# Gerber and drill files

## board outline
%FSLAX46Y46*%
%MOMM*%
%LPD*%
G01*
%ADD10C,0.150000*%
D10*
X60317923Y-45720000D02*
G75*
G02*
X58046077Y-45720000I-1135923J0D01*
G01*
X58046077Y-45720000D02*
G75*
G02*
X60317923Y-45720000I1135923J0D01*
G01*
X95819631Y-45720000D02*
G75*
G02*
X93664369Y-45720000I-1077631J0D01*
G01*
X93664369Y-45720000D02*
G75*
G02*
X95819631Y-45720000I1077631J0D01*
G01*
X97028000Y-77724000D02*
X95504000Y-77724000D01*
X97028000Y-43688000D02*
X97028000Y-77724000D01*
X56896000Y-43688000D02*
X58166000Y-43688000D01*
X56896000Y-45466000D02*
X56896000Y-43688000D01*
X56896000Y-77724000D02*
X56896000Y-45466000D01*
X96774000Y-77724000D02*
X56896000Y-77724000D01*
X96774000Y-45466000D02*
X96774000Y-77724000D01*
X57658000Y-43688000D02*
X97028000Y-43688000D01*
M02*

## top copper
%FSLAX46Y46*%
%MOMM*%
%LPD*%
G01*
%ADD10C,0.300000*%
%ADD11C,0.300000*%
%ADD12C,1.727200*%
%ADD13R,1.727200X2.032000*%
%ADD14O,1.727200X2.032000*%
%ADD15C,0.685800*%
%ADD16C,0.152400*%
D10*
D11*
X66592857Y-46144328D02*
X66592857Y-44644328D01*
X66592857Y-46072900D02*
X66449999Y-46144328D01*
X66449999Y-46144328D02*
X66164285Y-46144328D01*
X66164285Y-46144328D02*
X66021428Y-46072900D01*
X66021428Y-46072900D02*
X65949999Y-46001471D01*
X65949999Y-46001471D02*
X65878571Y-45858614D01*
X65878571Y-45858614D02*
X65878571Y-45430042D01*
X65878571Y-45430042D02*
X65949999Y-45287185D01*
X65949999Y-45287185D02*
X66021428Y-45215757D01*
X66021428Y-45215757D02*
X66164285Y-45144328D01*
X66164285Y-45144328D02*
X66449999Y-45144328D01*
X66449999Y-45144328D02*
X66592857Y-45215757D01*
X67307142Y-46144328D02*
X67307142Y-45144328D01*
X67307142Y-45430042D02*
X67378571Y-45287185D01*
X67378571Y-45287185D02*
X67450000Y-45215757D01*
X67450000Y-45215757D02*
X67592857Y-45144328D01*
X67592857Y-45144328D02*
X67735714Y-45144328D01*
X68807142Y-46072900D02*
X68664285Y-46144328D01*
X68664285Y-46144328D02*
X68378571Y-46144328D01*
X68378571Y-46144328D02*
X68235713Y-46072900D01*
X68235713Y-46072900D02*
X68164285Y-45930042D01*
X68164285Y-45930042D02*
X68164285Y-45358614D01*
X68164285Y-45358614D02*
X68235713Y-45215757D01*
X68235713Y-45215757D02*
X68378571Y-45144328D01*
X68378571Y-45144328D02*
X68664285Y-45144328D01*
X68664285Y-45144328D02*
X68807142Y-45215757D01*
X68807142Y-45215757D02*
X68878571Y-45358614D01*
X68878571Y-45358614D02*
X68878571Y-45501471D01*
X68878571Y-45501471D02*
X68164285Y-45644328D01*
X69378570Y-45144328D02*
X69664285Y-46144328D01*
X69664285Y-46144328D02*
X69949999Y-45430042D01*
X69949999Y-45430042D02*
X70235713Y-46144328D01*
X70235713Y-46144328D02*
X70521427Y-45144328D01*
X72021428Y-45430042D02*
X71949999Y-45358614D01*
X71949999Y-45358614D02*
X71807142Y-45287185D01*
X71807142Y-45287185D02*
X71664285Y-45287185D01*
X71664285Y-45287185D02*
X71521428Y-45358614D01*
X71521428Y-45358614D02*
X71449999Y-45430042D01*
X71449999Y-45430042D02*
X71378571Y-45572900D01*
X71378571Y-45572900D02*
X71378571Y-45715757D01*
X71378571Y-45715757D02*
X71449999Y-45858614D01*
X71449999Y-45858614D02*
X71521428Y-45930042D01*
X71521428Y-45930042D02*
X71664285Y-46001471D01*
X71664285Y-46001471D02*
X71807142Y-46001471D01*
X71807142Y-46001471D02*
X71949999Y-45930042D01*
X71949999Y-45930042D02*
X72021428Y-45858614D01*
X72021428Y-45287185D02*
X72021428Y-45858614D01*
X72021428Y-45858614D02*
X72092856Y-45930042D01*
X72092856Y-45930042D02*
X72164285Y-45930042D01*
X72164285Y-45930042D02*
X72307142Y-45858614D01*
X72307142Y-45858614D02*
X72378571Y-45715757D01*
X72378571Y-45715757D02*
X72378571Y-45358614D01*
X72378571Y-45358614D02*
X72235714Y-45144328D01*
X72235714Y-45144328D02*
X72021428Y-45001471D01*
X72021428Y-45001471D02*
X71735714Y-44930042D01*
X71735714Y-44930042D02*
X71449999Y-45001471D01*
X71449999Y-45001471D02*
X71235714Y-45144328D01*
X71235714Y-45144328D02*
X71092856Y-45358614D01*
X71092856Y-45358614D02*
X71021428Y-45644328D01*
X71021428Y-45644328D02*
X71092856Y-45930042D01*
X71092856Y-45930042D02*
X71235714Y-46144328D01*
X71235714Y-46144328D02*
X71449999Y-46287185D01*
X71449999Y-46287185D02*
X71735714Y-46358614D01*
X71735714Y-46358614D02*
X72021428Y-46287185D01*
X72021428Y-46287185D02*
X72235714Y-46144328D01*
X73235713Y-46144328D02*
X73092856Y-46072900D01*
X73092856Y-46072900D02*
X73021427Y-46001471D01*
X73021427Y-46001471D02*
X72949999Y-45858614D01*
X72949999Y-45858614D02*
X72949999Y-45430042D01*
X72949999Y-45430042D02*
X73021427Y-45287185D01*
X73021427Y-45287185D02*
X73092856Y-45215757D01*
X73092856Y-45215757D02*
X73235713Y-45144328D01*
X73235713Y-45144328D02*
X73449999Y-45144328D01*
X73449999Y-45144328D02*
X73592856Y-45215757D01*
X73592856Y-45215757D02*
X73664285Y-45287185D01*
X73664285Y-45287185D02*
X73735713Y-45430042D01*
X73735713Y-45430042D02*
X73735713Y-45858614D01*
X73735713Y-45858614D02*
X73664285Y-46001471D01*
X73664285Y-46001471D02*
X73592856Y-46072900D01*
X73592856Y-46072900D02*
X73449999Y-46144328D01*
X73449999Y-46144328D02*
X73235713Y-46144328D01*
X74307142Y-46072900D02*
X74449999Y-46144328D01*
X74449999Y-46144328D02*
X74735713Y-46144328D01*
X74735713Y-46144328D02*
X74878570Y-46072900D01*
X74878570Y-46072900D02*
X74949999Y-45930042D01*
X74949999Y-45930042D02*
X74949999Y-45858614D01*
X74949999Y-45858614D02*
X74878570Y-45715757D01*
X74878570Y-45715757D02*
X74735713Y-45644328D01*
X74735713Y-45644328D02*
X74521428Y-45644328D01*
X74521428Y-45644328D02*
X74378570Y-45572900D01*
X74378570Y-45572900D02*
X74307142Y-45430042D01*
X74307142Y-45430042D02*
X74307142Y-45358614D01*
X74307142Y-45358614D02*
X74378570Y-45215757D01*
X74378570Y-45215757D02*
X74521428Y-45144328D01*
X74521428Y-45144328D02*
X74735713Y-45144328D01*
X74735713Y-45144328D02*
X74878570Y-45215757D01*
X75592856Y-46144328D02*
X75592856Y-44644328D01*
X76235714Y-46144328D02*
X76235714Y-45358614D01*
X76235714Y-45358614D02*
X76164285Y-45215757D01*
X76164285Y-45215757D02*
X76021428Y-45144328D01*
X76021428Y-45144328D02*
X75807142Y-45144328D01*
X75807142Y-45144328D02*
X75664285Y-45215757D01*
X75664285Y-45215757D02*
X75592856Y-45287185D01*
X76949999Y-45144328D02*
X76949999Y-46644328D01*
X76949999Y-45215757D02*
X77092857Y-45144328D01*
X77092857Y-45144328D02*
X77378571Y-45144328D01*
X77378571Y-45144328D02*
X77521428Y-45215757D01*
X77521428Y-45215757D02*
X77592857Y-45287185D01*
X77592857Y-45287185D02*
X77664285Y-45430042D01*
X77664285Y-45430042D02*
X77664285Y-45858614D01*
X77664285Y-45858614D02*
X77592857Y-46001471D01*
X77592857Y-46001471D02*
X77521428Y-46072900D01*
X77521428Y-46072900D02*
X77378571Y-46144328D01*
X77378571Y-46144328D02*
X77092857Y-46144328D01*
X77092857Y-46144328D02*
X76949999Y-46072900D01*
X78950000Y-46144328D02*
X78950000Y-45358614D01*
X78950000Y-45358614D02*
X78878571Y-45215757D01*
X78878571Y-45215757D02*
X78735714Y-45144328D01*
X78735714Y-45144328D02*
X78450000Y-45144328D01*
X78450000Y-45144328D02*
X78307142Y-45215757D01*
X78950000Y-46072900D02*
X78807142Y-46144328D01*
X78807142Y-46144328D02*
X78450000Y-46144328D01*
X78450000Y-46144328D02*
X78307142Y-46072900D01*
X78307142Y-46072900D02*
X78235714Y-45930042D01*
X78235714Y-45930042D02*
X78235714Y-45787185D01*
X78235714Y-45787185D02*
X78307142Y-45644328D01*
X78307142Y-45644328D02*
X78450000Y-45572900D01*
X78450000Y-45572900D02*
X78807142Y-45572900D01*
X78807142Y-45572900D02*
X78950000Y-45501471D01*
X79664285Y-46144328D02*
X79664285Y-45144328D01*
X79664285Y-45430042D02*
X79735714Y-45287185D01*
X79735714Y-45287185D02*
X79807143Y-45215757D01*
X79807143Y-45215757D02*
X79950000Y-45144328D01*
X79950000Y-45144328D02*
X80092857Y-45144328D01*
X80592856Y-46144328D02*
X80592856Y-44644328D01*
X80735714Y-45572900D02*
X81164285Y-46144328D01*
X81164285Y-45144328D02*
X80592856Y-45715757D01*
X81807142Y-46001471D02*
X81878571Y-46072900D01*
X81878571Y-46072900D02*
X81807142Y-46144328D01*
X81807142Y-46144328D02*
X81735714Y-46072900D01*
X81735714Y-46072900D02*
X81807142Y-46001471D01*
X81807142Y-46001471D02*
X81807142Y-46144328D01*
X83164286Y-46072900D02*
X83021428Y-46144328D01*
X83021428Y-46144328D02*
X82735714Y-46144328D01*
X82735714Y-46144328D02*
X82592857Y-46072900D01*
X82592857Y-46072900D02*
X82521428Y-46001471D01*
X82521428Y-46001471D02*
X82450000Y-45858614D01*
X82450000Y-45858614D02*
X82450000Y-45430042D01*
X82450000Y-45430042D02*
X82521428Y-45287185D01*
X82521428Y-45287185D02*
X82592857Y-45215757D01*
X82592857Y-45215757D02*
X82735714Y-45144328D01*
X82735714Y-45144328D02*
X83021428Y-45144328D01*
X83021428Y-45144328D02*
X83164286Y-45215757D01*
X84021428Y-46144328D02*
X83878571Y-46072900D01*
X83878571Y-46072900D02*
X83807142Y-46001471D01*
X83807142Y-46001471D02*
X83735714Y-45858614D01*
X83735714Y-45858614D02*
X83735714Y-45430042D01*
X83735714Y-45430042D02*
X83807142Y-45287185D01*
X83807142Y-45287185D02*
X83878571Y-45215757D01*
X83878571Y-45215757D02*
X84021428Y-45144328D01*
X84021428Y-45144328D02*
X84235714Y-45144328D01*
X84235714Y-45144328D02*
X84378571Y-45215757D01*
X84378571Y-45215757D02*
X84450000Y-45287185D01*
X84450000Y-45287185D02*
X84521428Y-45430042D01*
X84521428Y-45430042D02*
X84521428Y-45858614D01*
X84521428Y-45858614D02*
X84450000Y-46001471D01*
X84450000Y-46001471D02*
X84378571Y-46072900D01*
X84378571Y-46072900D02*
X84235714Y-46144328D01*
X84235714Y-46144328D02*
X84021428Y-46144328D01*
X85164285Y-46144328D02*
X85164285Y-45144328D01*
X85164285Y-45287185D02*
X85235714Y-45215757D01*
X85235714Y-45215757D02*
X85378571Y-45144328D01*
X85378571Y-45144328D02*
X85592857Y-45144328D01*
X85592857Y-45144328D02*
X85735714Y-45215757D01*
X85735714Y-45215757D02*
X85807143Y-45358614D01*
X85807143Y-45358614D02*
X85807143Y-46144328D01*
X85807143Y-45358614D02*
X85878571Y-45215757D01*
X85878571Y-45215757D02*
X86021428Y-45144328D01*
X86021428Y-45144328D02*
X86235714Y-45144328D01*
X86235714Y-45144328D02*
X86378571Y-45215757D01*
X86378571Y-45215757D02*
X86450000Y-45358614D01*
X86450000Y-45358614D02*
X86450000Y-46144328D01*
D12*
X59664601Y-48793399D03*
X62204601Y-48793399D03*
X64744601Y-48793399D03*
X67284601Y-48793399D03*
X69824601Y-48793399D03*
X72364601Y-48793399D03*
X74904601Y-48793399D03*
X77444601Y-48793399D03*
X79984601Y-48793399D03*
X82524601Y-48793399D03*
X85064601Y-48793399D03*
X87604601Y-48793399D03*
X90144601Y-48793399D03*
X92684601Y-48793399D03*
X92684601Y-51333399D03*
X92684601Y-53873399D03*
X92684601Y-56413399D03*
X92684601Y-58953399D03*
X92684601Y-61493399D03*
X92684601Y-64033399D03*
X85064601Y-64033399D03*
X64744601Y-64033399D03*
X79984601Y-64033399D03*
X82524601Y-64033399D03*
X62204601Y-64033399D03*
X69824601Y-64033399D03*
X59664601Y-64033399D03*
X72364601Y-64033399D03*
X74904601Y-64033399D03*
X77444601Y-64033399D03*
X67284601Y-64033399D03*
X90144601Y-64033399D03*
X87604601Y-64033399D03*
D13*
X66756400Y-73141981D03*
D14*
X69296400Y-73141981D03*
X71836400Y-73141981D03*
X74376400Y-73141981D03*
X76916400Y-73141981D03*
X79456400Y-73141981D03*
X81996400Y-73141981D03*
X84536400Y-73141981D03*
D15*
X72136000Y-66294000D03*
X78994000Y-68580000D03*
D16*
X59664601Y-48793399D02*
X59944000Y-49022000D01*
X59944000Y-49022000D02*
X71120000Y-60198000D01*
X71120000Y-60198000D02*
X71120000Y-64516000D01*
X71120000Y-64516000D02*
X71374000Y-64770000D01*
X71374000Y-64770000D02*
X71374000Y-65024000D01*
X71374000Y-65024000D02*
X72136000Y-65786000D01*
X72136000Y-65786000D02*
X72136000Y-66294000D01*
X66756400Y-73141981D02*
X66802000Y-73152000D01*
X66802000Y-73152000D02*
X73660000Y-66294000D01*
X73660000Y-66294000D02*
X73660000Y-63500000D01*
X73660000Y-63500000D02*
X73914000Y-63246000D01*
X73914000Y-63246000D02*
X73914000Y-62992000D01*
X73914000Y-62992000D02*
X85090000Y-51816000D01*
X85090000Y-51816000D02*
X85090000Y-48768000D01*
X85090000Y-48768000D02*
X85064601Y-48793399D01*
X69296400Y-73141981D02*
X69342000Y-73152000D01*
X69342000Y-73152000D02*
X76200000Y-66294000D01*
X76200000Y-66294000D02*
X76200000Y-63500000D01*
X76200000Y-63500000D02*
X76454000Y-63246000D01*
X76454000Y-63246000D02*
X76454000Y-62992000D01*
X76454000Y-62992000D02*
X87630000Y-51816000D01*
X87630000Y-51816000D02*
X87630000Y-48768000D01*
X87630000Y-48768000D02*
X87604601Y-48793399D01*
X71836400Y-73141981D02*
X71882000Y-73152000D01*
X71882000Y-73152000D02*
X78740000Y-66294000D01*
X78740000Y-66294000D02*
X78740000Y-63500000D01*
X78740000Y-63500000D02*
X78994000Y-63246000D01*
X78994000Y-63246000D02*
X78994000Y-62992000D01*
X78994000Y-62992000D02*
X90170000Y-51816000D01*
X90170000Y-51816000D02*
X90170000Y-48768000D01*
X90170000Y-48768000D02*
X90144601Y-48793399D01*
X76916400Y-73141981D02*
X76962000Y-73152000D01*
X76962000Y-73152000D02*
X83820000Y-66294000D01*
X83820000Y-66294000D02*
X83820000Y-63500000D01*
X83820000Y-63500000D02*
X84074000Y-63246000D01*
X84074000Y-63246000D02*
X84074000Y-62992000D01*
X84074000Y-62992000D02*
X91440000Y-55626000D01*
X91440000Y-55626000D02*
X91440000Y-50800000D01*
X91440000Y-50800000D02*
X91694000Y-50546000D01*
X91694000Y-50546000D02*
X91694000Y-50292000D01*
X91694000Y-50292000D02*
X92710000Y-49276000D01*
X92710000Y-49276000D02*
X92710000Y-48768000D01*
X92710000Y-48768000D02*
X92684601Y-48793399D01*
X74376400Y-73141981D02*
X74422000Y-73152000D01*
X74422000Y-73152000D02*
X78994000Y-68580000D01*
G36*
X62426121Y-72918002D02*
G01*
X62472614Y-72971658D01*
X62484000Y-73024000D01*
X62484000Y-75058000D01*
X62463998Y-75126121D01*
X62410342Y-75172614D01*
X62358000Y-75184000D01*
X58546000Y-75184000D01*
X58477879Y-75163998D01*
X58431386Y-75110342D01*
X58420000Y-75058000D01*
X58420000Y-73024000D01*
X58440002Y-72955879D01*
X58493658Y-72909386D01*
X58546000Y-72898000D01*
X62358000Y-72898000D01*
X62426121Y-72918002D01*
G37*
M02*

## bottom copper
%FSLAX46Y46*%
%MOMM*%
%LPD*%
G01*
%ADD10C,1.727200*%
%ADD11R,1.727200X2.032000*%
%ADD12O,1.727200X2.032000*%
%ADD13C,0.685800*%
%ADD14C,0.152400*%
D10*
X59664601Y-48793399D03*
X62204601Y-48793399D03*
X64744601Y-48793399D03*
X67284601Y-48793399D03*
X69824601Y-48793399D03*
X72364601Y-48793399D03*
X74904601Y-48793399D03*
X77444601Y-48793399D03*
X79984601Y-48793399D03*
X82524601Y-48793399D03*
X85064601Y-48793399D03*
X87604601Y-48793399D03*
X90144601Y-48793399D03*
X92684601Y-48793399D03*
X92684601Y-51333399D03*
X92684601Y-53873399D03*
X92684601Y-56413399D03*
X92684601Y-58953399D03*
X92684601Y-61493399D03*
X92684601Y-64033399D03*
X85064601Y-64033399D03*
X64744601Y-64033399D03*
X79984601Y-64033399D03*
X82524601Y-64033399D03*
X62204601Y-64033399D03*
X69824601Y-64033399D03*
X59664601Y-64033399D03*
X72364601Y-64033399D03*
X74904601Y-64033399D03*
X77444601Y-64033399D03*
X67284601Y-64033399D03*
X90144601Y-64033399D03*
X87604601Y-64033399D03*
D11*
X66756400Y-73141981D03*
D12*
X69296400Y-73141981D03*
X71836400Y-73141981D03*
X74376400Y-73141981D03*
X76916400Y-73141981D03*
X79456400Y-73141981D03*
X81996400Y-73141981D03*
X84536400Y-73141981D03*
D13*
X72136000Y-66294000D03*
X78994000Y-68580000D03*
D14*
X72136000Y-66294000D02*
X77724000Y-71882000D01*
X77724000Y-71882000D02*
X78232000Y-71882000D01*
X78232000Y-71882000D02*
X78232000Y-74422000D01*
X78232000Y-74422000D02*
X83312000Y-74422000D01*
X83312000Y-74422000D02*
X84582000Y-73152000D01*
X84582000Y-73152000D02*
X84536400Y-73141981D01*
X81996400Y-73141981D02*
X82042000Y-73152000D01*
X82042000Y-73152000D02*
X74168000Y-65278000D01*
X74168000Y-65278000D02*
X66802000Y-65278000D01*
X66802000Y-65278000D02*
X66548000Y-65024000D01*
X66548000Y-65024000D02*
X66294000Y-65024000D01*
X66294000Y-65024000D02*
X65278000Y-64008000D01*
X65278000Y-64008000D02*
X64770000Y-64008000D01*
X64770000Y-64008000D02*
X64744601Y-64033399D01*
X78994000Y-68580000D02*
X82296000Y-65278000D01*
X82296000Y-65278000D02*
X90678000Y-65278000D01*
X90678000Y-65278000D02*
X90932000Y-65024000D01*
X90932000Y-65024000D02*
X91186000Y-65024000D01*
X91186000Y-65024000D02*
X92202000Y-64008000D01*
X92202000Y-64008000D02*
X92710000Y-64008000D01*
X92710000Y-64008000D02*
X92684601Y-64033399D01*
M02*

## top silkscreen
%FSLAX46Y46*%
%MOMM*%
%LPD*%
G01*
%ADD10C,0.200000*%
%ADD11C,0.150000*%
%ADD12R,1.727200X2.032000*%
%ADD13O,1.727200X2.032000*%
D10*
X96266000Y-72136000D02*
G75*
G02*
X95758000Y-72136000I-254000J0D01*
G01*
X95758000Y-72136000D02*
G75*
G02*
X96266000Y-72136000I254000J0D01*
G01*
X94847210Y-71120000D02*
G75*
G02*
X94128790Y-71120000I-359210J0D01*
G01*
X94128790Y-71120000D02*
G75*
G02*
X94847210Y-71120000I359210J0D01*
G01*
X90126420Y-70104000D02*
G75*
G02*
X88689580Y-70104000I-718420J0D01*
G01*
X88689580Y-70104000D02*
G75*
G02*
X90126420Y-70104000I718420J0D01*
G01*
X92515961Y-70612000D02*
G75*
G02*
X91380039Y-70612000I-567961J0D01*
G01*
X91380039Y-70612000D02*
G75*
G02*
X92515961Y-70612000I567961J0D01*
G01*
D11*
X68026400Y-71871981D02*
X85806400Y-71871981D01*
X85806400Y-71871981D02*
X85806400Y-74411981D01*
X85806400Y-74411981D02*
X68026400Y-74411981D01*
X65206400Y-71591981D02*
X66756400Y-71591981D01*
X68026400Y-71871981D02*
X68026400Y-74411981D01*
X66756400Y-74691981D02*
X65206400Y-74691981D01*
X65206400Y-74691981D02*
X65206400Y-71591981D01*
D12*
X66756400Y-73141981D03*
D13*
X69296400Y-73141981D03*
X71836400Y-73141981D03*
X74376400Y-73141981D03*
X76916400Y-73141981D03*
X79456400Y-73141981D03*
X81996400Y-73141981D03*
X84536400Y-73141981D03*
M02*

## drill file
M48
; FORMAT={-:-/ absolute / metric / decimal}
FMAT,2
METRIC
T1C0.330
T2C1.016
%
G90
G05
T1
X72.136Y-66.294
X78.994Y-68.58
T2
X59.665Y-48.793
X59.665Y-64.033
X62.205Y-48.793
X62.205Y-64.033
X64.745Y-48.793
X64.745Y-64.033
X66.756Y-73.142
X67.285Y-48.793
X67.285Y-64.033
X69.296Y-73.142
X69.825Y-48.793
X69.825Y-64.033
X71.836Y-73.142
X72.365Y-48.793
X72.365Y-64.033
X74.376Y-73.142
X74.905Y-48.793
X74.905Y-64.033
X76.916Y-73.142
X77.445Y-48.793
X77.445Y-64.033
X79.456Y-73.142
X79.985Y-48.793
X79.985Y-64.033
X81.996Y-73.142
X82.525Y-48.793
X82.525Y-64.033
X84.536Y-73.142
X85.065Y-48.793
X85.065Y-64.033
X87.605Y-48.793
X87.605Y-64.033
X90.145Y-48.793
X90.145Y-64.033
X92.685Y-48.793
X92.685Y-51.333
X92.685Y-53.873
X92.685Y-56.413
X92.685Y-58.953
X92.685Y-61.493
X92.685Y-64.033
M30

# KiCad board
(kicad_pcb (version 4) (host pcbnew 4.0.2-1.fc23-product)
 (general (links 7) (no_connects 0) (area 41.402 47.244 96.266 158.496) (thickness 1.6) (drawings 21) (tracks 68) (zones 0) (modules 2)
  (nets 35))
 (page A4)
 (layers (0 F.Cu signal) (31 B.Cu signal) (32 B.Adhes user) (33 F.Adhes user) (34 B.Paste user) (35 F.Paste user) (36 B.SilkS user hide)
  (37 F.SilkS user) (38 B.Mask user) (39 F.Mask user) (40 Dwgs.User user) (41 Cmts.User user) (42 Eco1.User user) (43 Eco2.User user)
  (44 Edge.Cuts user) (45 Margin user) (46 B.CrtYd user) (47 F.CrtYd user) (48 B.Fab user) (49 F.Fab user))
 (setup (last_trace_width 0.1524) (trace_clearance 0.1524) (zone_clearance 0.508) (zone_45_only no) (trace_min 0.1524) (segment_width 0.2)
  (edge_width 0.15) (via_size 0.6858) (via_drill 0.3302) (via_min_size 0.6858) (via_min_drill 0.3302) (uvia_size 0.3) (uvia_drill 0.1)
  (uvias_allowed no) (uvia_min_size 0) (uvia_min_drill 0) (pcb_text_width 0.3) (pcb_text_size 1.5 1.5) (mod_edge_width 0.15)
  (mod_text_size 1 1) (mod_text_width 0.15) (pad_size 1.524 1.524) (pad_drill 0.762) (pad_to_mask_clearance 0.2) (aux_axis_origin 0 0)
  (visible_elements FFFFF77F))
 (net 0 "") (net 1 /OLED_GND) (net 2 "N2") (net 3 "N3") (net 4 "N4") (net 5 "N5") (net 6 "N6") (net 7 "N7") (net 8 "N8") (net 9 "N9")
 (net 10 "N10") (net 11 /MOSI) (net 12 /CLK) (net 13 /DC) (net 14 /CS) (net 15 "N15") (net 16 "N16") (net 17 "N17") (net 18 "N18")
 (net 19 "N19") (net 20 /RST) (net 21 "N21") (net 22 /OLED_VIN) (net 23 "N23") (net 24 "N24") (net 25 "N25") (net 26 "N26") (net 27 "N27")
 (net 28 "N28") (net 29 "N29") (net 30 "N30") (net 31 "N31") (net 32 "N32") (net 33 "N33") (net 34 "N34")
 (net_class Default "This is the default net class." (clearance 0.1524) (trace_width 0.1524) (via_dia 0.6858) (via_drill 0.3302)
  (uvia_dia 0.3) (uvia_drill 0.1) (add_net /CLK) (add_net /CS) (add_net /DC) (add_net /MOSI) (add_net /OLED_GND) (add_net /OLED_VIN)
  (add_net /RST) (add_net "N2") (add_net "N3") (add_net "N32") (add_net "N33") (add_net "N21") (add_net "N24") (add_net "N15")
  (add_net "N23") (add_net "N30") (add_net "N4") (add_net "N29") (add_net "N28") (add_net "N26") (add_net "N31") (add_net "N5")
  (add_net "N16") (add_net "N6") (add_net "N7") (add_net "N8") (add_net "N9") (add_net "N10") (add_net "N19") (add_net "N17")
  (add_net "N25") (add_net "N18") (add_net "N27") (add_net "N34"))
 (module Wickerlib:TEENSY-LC (layer B.Cu) (at 69.824601 58.953399 270)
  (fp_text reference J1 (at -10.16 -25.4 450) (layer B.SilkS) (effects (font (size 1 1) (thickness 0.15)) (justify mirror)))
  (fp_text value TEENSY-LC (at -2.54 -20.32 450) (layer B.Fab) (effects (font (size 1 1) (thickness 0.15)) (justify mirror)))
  (pad G1 thru_hole circle (at -10.16 10.16 270) (size 1.7272 1.7272) (drill 1.016) (layers *.Cu *.Mask B.SilkS) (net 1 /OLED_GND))
  (pad 0 thru_hole circle (at -10.16 7.62 270) (size 1.7272 1.7272) (drill 1.016) (layers *.Cu *.Mask B.SilkS) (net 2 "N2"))
  (pad 1 thru_hole circle (at -10.16 5.08 270) (size 1.7272 1.7272) (drill 1.016) (layers *.Cu *.Mask B.SilkS) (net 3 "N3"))
  (pad 2 thru_hole circle (at -10.16 2.54 270) (size 1.7272 1.7272) (drill 1.016) (layers *.Cu *.Mask B.SilkS) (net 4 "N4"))
  (pad 3 thru_hole circle (at -10.16 0 270) (size 1.7272 1.7272) (drill 1.016) (layers *.Cu *.Mask B.SilkS) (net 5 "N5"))
  (pad 4 thru_hole circle (at -10.16 -2.54 270) (size 1.7272 1.7272) (drill 1.016) (layers *.Cu *.Mask B.SilkS) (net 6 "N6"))
  (pad 5 thru_hole circle (at -10.16 -5.08 270) (size 1.7272 1.7272) (drill 1.016) (layers *.Cu *.Mask B.SilkS) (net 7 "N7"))
  (pad 6 thru_hole circle (at -10.16 -7.62 270) (size 1.7272 1.7272) (drill 1.016) (layers *.Cu *.Mask B.SilkS) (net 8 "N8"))
  (pad 7 thru_hole circle (at -10.16 -10.16 270) (size 1.7272 1.7272) (drill 1.016) (layers *.Cu *.Mask B.SilkS) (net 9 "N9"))
  (pad 8 thru_hole circle (at -10.16 -12.7 270) (size 1.7272 1.7272) (drill 1.016) (layers *.Cu *.Mask B.SilkS) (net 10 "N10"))
  (pad 9 thru_hole circle (at -10.16 -15.24 270) (size 1.7272 1.7272) (drill 1.016) (layers *.Cu *.Mask B.SilkS) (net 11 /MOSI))
  (pad 10 thru_hole circle (at -10.16 -17.78 270) (size 1.7272 1.7272) (drill 1.016) (layers *.Cu *.Mask B.SilkS) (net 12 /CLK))
  (pad 11 thru_hole circle (at -10.16 -20.32 270) (size 1.7272 1.7272) (drill 1.016) (layers *.Cu *.Mask B.SilkS) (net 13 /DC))
  (pad 12 thru_hole circle (at -10.16 -22.86 270) (size 1.7272 1.7272) (drill 1.016) (layers *.Cu *.Mask B.SilkS) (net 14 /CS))
  (pad 17A thru_hole circle (at -7.62 -22.86 270) (size 1.7272 1.7272) (drill 1.016) (layers *.Cu *.Mask B.SilkS) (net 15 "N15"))
  (pad 3V1 thru_hole circle (at -5.08 -22.86 270) (size 1.7272 1.7272) (drill 1.016) (layers *.Cu *.Mask B.SilkS) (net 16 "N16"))
  (pad G2 thru_hole circle (at -2.54 -22.86 270) (size 1.7272 1.7272) (drill 1.016) (layers *.Cu *.Mask B.SilkS) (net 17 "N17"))
  (pad PGM thru_hole circle (at 0 -22.86 270) (size 1.7272 1.7272) (drill 1.016) (layers *.Cu *.Mask B.SilkS) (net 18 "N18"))
  (pad DAC thru_hole circle (at 2.54 -22.86 270) (size 1.7272 1.7272) (drill 1.016) (layers *.Cu *.Mask B.SilkS) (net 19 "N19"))
  (pad 13 thru_hole circle (at 5.08 -22.86 270) (size 1.7272 1.7272) (drill 1.016) (layers *.Cu *.Mask B.SilkS) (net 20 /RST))
  (pad 16 thru_hole circle (at 5.08 -15.24 270) (size 1.7272 1.7272) (drill 1.016) (layers *.Cu *.Mask B.SilkS) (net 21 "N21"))
  (pad 3V2 thru_hole circle (at 5.08 5.08 270) (size 1.7272 1.7272) (drill 1.016) (layers *.Cu *.Mask B.SilkS) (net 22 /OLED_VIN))
  (pad 18 thru_hole circle (at 5.08 -10.16 270) (size 1.7272 1.7272) (drill 1.016) (layers *.Cu *.Mask B.SilkS) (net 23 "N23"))
  (pad 17 thru_hole circle (at 5.08 -12.7 270) (size 1.7272 1.7272) (drill 1.016) (layers *.Cu *.Mask B.SilkS) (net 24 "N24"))
  (pad G3 thru_hole circle (at 5.08 7.62 270) (size 1.7272 1.7272) (drill 1.016) (layers *.Cu *.Mask B.SilkS) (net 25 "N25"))
  (pad 22 thru_hole circle (at 5.08 0 270) (size 1.7272 1.7272) (drill 1.016) (layers *.Cu *.Mask B.SilkS) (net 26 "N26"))
  (pad VIN thru_hole circle (at 5.08 10.16 270) (size 1.7272 1.7272) (drill 1.016) (layers *.Cu *.Mask B.SilkS) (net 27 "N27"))
  (pad 21 thru_hole circle (at 5.08 -2.54 270) (size 1.7272 1.7272) (drill 1.016) (layers *.Cu *.Mask B.SilkS) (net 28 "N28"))
  (pad 20 thru_hole circle (at 5.08 -5.08 270) (size 1.7272 1.7272) (drill 1.016) (layers *.Cu *.Mask B.SilkS) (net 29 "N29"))
  (pad 19 thru_hole circle (at 5.08 -7.62 270) (size 1.7272 1.7272) (drill 1.016) (layers *.Cu *.Mask B.SilkS) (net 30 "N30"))
  (pad 23 thru_hole circle (at 5.08 2.54 270) (size 1.7272 1.7272) (drill 1.016) (layers *.Cu *.Mask B.SilkS) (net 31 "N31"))
  (pad 14 thru_hole circle (at 5.08 -20.32 270) (size 1.7272 1.7272) (drill 1.016) (layers *.Cu *.Mask B.SilkS) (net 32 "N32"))
  (pad 15 thru_hole circle (at 5.08 -17.78 270) (size 1.7272 1.7272) (drill 1.016) (layers *.Cu *.Mask B.SilkS) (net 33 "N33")))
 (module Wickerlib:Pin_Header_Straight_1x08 (layer F.Cu) (at 66.7564 73.141981 90)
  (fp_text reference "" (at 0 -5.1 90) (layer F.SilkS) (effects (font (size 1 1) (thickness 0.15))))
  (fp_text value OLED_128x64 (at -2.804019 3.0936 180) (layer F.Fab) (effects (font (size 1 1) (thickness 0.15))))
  (fp_line (start 1.27 1.27) (end 1.27 19.05) (layer F.SilkS) (width 0.15))
  (fp_line (start 1.27 19.05) (end -1.27 19.05) (layer F.SilkS) (width 0.15))
  (fp_line (start -1.27 19.05) (end -1.27 1.27) (layer F.SilkS) (width 0.15))
  (fp_line (start 1.55 -1.55) (end 1.55 0) (layer F.SilkS) (width 0.15))
  (fp_line (start 1.27 1.27) (end -1.27 1.27) (layer F.SilkS) (width 0.15))
  (fp_line (start -1.55 0) (end -1.55 -1.55) (layer F.SilkS) (width 0.15))
  (fp_line (start -1.55 -1.55) (end 1.55 -1.55) (layer F.SilkS) (width 0.15))
  (pad 1 thru_hole rect (at 0 0 90) (size 2.032 1.7272) (drill 1.016) (layers *.Cu *.Mask F.SilkS) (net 11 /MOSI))
  (pad 2 thru_hole oval (at 0 2.54 90) (size 2.032 1.7272) (drill 1.016) (layers *.Cu *.Mask F.SilkS) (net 12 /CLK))
  (pad 3 thru_hole oval (at 0 5.08 90) (size 2.032 1.7272) (drill 1.016) (layers *.Cu *.Mask F.SilkS) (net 13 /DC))
  (pad 4 thru_hole oval (at 0 7.62 90) (size 2.032 1.7272) (drill 1.016) (layers *.Cu *.Mask F.SilkS) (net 20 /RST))
  (pad 5 thru_hole oval (at 0 10.16 90) (size 2.032 1.7272) (drill 1.016) (layers *.Cu *.Mask F.SilkS) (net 14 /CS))
  (pad 6 thru_hole oval (at 0 12.7 90) (size 2.032 1.7272) (drill 1.016) (layers *.Cu *.Mask F.SilkS) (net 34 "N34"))
  (pad 7 thru_hole oval (at 0 15.24 90) (size 2.032 1.7272) (drill 1.016) (layers *.Cu *.Mask F.SilkS) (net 22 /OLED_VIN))
  (pad 8 thru_hole oval (at 0 17.78 90) (size 2.032 1.7272) (drill 1.016) (layers *.Cu *.Mask F.SilkS) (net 1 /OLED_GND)))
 (gr_circle (center 96.012 72.136) (end 95.758 72.136) (layer F.SilkS) (width 0.2))
 (gr_circle (center 94.488 71.12) (end 94.234 70.866) (layer F.SilkS) (width 0.2))
 (gr_circle (center 89.408 70.104) (end 89.916 70.612) (layer F.SilkS) (width 0.2))
 (gr_circle (center 91.948 70.612) (end 91.694 70.104) (layer F.SilkS) (width 0.2))
 (gr_circle (center 59.182 45.72) (end 58.166 45.212) (layer Edge.Cuts) (width 0.15))
 (gr_circle (center 94.742 45.72) (end 93.98 44.958) (layer Edge.Cuts) (width 0.15))
 (gr_line (start 97.028 77.724) (end 95.504 77.724) (angle 90) (layer Edge.Cuts) (width 0.15))
 (gr_line (start 97.028 43.688) (end 97.028 77.724) (angle 90) (layer Edge.Cuts) (width 0.15))
 (gr_line (start 56.896 43.688) (end 58.166 43.688) (angle 90) (layer Edge.Cuts) (width 0.15))
 (gr_line (start 56.896 45.466) (end 56.896 43.688) (angle 90) (layer Edge.Cuts) (width 0.15))
 (gr_line (start 56.896 77.724) (end 56.896 45.466) (angle 90) (layer Edge.Cuts) (width 0.15))
 (gr_line (start 96.774 77.724) (end 56.896 77.724) (angle 90) (layer Edge.Cuts) (width 0.15))
 (gr_line (start 96.774 45.466) (end 96.774 77.724) (angle 90) (layer Edge.Cuts) (width 0.15))
 (gr_line (start 57.658 43.688) (end 97.028 43.688) (angle 90) (layer Edge.Cuts) (width 0.15))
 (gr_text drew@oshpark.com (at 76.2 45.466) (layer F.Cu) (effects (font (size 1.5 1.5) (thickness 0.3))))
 (segment (start 59.664601 48.793399) (end 59.944 49.022) (width 0.1524) (layer F.Cu) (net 1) (status 80000))
 (segment (start 59.944 49.022) (end 71.12 60.198) (width 0.1524) (layer F.Cu) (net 1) (status 80000))
 (segment (start 71.12 60.198) (end 71.12 64.516) (width 0.1524) (layer F.Cu) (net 1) (status 80000))
 (segment (start 71.12 64.516) (end 71.374 64.77) (width 0.1524) (layer F.Cu) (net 1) (status 80000))
 (segment (start 71.374 64.77) (end 71.374 65.024) (width 0.1524) (layer F.Cu) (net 1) (status 80000))
 (segment (start 71.374 65.024) (end 72.136 65.786) (width 0.1524) (layer F.Cu) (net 1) (status 80000))
 (segment (start 72.136 65.786) (end 72.136 66.294) (width 0.1524) (layer F.Cu) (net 1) (status 80000))
 (via (at 72.136 66.294) (size 0.6858) (layers F.Cu B.Cu) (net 1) (status 80000))
 (segment (start 72.136 66.294) (end 77.724 71.882) (width 0.1524) (layer B.Cu) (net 1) (status 80000))
 (segment (start 77.724 71.882) (end 78.232 71.882) (width 0.1524) (layer B.Cu) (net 1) (status 80000))
 (segment (start 78.232 71.882) (end 78.232 74.422) (width 0.1524) (layer B.Cu) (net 1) (status 80000))
 (segment (start 78.232 74.422) (end 83.312 74.422) (width 0.1524) (layer B.Cu) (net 1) (status 80000))
 (segment (start 83.312 74.422) (end 84.582 73.152) (width 0.1524) (layer B.Cu) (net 1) (status 80000))
 (segment (start 84.582 73.152) (end 84.5364 73.141981) (width 0.1524) (layer B.Cu) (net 1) (status 80000))
 (segment (start 66.7564 73.141981) (end 66.802 73.152) (width 0.1524) (layer F.Cu) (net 11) (status 80000))
 (segment (start 66.802 73.152) (end 73.66 66.294) (width 0.1524) (layer F.Cu) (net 11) (status 80000))
 (segment (start 73.66 66.294) (end 73.66 63.5) (width 0.1524) (layer F.Cu) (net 11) (status 80000))
 (segment (start 73.66 63.5) (end 73.914 63.246) (width 0.1524) (layer F.Cu) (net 11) (status 80000))
 (segment (start 73.914 63.246) (end 73.914 62.992) (width 0.1524) (layer F.Cu) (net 11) (status 80000))
 (segment (start 73.914 62.992) (end 85.09 51.816) (width 0.1524) (layer F.Cu) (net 11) (status 80000))
 (segment (start 85.09 51.816) (end 85.09 48.768) (width 0.1524) (layer F.Cu) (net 11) (status 80000))
 (segment (start 85.09 48.768) (end 85.064601 48.793399) (width 0.1524) (layer F.Cu) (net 11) (status 80000))
 (segment (start 69.2964 73.141981) (end 69.342 73.152) (width 0.1524) (layer F.Cu) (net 12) (status 80000))
 (segment (start 69.342 73.152) (end 76.2 66.294) (width 0.1524) (layer F.Cu) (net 12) (status 80000))
 (segment (start 76.2 66.294) (end 76.2 63.5) (width 0.1524) (layer F.Cu) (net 12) (status 80000))
 (segment (start 76.2 63.5) (end 76.454 63.246) (width 0.1524) (layer F.Cu) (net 12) (status 80000))
 (segment (start 76.454 63.246) (end 76.454 62.992) (width 0.1524) (layer F.Cu) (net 12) (status 80000))
 (segment (start 76.454 62.992) (end 87.63 51.816) (width 0.1524) (layer F.Cu) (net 12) (status 80000))
 (segment (start 87.63 51.816) (end 87.63 48.768) (width 0.1524) (layer F.Cu) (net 12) (status 80000))
 (segment (start 87.63 48.768) (end 87.604601 48.793399) (width 0.1524) (layer F.Cu) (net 12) (status 80000))
 (segment (start 71.8364 73.141981) (end 71.882 73.152) (width 0.1524) (layer F.Cu) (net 13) (status 80000))
 (segment (start 71.882 73.152) (end 78.74 66.294) (width 0.1524) (layer F.Cu) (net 13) (status 80000))
 (segment (start 78.74 66.294) (end 78.74 63.5) (width 0.1524) (layer F.Cu) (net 13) (status 80000))
 (segment (start 78.74 63.5) (end 78.994 63.246) (width 0.1524) (layer F.Cu) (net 13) (status 80000))
 (segment (start 78.994 63.246) (end 78.994 62.992) (width 0.1524) (layer F.Cu) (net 13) (status 80000))
 (segment (start 78.994 62.992) (end 90.17 51.816) (width 0.1524) (layer F.Cu) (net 13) (status 80000))
 (segment (start 90.17 51.816) (end 90.17 48.768) (width 0.1524) (layer F.Cu) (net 13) (status 80000))
 (segment (start 90.17 48.768) (end 90.144601 48.793399) (width 0.1524) (layer F.Cu) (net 13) (status 80000))
 (segment (start 76.9164 73.141981) (end 76.962 73.152) (width 0.1524) (layer F.Cu) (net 14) (status 80000))
 (segment (start 76.962 73.152) (end 83.82 66.294) (width 0.1524) (layer F.Cu) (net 14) (status 80000))
 (segment (start 83.82 66.294) (end 83.82 63.5) (width 0.1524) (layer F.Cu) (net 14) (status 80000))
 (segment (start 83.82 63.5) (end 84.074 63.246) (width 0.1524) (layer F.Cu) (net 14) (status 80000))
 (segment (start 84.074 63.246) (end 84.074 62.992) (width 0.1524) (layer F.Cu) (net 14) (status 80000))
 (segment (start 84.074 62.992) (end 91.44 55.626) (width 0.1524) (layer F.Cu) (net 14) (status 80000))
 (segment (start 91.44 55.626) (end 91.44 50.8) (width 0.1524) (layer F.Cu) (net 14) (status 80000))
 (segment (start 91.44 50.8) (end 91.694 50.546) (width 0.1524) (layer F.Cu) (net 14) (status 80000))
 (segment (start 91.694 50.546) (end 91.694 50.292) (width 0.1524) (layer F.Cu) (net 14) (status 80000))
 (segment (start 91.694 50.292) (end 92.71 49.276) (width 0.1524) (layer F.Cu) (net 14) (status 80000))
 (segment (start 92.71 49.276) (end 92.71 48.768) (width 0.1524) (layer F.Cu) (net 14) (status 80000))
 (segment (start 92.71 48.768) (end 92.684601 48.793399) (width 0.1524) (layer F.Cu) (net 14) (status 80000))
 (segment (start 81.9964 73.141981) (end 82.042 73.152) (width 0.1524) (layer B.Cu) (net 22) (status 80000))
 (segment (start 82.042 73.152) (end 74.168 65.278) (width 0.1524) (layer B.Cu) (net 22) (status 80000))
 (segment (start 74.168 65.278) (end 66.802 65.278) (width 0.1524) (layer B.Cu) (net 22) (status 80000))
 (segment (start 66.802 65.278) (end 66.548 65.024) (width 0.1524) (layer B.Cu) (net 22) (status 80000))
 (segment (start 66.548 65.024) (end 66.294 65.024) (width 0.1524) (layer B.Cu) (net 22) (status 80000))
 (segment (start 66.294 65.024) (end 65.278 64.008) (width 0.1524) (layer B.Cu) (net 22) (status 80000))
 (segment (start 65.278 64.008) (end 64.77 64.008) (width 0.1524) (layer B.Cu) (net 22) (status 80000))
 (segment (start 64.77 64.008) (end 64.744601 64.033399) (width 0.1524) (layer B.Cu) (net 22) (status 80000))
 (segment (start 74.3764 73.141981) (end 74.422 73.152) (width 0.1524) (layer F.Cu) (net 20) (status 80000))
 (segment (start 74.422 73.152) (end 78.994 68.58) (width 0.1524) (layer F.Cu) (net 20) (status 80000))
 (via (at 78.994 68.58) (size 0.6858) (layers F.Cu B.Cu) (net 20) (status 80000))
 (segment (start 78.994 68.58) (end 82.296 65.278) (width 0.1524) (layer B.Cu) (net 20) (status 80000))
 (segment (start 82.296 65.278) (end 90.678 65.278) (width 0.1524) (layer B.Cu) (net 20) (status 80000))
 (segment (start 90.678 65.278) (end 90.932 65.024) (width 0.1524) (layer B.Cu) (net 20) (status 80000))
 (segment (start 90.932 65.024) (end 91.186 65.024) (width 0.1524) (layer B.Cu) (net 20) (status 80000))
 (segment (start 91.186 65.024) (end 92.202 64.008) (width 0.1524) (layer B.Cu) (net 20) (status 80000))
 (segment (start 92.202 64.008) (end 92.71 64.008) (width 0.1524) (layer B.Cu) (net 20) (status 80000))
 (segment (start 92.71 64.008) (end 92.684601 64.033399) (width 0.1524) (layer B.Cu) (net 20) (status 80000))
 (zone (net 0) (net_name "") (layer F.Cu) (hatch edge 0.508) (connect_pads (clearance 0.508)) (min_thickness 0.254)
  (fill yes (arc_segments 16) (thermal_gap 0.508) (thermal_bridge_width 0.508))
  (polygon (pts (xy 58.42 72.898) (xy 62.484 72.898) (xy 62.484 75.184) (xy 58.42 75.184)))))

